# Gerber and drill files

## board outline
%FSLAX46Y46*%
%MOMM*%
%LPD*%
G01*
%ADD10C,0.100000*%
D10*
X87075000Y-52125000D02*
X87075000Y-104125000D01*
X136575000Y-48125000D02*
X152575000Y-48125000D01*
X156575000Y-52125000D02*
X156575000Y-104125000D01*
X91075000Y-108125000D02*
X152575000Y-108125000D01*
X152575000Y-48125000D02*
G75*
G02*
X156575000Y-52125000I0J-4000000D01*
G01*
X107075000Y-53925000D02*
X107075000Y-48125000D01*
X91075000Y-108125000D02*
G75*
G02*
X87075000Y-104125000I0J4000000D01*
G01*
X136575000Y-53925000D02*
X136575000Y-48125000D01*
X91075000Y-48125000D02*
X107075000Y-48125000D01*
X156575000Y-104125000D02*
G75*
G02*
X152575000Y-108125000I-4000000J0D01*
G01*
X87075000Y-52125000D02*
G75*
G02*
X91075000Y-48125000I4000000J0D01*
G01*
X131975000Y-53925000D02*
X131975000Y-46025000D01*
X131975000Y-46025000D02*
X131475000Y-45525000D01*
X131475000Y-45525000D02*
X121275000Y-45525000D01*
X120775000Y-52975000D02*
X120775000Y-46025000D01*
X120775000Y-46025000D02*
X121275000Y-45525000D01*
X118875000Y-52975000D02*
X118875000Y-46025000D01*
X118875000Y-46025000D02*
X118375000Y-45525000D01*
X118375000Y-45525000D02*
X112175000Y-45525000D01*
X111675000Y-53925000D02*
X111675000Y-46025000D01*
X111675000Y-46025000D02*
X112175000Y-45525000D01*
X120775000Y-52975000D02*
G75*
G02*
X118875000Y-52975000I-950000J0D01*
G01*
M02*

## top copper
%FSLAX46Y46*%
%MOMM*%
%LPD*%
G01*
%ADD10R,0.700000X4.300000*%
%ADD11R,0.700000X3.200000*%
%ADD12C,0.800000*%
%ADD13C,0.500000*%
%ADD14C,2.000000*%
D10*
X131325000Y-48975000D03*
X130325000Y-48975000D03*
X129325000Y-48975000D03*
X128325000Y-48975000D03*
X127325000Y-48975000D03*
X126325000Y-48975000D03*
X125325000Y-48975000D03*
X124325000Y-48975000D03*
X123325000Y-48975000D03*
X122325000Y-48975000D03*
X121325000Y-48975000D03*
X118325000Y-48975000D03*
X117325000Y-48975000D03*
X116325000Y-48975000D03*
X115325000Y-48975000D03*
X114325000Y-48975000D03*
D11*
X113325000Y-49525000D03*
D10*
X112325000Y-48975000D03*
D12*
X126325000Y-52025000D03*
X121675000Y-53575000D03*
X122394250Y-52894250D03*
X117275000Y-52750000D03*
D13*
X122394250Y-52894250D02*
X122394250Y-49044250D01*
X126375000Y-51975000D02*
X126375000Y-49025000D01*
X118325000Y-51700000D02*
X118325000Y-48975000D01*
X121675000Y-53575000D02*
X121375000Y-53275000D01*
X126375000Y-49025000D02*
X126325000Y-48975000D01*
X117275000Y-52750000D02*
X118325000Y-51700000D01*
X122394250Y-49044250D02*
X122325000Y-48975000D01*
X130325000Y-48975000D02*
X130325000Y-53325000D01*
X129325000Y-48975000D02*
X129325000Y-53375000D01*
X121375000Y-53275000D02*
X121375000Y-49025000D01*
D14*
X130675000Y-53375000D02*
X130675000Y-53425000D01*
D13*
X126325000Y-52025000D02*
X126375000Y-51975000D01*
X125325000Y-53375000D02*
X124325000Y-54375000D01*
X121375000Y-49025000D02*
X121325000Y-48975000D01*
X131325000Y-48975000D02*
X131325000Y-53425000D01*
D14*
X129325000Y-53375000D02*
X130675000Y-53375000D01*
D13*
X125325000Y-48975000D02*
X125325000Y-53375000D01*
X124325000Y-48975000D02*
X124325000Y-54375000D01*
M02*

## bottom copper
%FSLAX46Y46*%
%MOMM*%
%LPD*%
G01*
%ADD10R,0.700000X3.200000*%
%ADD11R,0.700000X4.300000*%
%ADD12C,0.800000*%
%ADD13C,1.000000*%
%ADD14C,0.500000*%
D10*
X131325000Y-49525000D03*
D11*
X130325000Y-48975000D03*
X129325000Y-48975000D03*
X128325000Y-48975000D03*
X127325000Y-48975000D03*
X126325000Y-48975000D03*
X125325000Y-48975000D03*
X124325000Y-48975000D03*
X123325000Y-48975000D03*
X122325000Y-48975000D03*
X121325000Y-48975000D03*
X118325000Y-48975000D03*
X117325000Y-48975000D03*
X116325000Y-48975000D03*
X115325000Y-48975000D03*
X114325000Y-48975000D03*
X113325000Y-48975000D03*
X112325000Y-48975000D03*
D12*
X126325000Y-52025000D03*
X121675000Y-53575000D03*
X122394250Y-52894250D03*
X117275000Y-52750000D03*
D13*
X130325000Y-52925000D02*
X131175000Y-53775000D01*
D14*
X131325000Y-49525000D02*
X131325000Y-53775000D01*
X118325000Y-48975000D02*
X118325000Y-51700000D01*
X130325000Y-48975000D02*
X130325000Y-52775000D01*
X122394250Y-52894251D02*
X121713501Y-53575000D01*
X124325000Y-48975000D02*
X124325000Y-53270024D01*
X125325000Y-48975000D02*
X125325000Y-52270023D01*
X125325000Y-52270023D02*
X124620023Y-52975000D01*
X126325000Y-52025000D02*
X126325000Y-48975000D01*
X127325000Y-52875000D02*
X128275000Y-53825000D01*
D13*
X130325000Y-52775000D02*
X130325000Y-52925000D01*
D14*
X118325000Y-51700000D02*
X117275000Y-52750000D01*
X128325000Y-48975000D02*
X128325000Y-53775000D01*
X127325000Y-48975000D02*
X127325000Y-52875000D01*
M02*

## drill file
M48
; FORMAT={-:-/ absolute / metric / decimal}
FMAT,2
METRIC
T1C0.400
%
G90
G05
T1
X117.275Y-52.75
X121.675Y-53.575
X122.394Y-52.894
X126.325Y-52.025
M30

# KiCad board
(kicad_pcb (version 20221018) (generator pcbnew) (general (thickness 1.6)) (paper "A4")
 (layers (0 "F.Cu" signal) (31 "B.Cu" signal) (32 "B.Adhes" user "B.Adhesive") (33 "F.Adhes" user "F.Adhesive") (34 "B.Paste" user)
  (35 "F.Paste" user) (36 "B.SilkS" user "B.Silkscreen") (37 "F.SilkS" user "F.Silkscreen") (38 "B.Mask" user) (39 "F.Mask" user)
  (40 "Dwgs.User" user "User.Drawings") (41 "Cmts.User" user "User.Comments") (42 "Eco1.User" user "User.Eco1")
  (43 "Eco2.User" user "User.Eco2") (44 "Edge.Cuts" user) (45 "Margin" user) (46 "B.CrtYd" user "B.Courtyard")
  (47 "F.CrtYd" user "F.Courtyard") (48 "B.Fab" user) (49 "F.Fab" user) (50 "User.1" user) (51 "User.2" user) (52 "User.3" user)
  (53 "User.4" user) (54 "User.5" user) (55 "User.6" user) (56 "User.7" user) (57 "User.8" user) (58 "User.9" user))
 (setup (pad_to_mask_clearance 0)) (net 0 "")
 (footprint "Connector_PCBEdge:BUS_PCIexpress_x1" (layer "F.Cu") (at 131.325 48.975 180)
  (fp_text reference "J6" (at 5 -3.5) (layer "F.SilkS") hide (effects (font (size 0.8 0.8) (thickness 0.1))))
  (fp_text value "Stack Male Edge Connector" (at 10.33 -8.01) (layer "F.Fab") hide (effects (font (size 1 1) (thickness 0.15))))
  (fp_line (start -0.65 -4.95) (end -0.65 2.95) (stroke (width 0.1) (type solid)) (layer "Edge.Cuts"))
  (fp_line (start -0.65 2.95) (end -0.15 3.45) (stroke (width 0.1) (type solid)) (layer "Edge.Cuts"))
  (fp_line (start -0.15 3.45) (end 10.05 3.45) (stroke (width 0.1) (type solid)) (layer "Edge.Cuts"))
  (fp_line (start 10.55 -4) (end 10.55 2.95) (stroke (width 0.1) (type solid)) (layer "Edge.Cuts"))
  (fp_line (start 10.55 2.95) (end 10.05 3.45) (stroke (width 0.1) (type solid)) (layer "Edge.Cuts"))
  (fp_line (start 12.45 -4) (end 12.45 2.95) (stroke (width 0.1) (type solid)) (layer "Edge.Cuts"))
  (fp_line (start 12.45 2.95) (end 12.95 3.45) (stroke (width 0.1) (type solid)) (layer "Edge.Cuts"))
  (fp_line (start 12.95 3.45) (end 19.15 3.45) (stroke (width 0.1) (type solid)) (layer "Edge.Cuts"))
  (fp_line (start 19.65 -4.95) (end 19.65 2.95) (stroke (width 0.1) (type solid)) (layer "Edge.Cuts"))
  (fp_line (start 19.65 2.95) (end 19.15 3.45) (stroke (width 0.1) (type solid)) (layer "Edge.Cuts"))
  (fp_arc (start 10.55 -4) (mid 11.5 -4.95) (end 12.45 -4) (stroke (width 0.1) (type solid)) (layer "Edge.Cuts"))
  (pad "A1" connect rect (at 0 -0.55 180) (size 0.7 3.2) (layers "B.Cu" "B.Mask"))
  (pad "A2" connect rect (at 1 0 180) (size 0.7 4.3) (layers "B.Cu" "B.Mask"))
  (pad "A3" connect rect (at 2 0 180) (size 0.7 4.3) (layers "B.Cu" "B.Mask"))
  (pad "A4" connect rect (at 3 0 180) (size 0.7 4.3) (layers "B.Cu" "B.Mask"))
  (pad "A5" connect rect (at 4 0 180) (size 0.7 4.3) (layers "B.Cu" "B.Mask"))
  (pad "A6" connect rect (at 5 0 180) (size 0.7 4.3) (layers "B.Cu" "B.Mask"))
  (pad "A7" connect rect (at 6 0 180) (size 0.7 4.3) (layers "B.Cu" "B.Mask"))
  (pad "A8" connect rect (at 7 0 180) (size 0.7 4.3) (layers "B.Cu" "B.Mask"))
  (pad "A9" connect rect (at 8 0 180) (size 0.7 4.3) (layers "B.Cu" "B.Mask"))
  (pad "A10" connect rect (at 9 0 180) (size 0.7 4.3) (layers "B.Cu" "B.Mask"))
  (pad "A11" connect rect (at 10 0 180) (size 0.7 4.3) (layers "B.Cu" "B.Mask"))
  (pad "A12" connect rect (at 13 0 180) (size 0.7 4.3) (layers "B.Cu" "B.Mask"))
  (pad "A13" connect rect (at 14 0 180) (size 0.7 4.3) (layers "B.Cu" "B.Mask"))
  (pad "A14" connect rect (at 15 0 180) (size 0.7 4.3) (layers "B.Cu" "B.Mask"))
  (pad "A15" connect rect (at 16 0 180) (size 0.7 4.3) (layers "B.Cu" "B.Mask"))
  (pad "A16" connect rect (at 17 0 180) (size 0.7 4.3) (layers "B.Cu" "B.Mask"))
  (pad "A17" connect rect (at 18 0 180) (size 0.7 4.3) (layers "B.Cu" "B.Mask"))
  (pad "A18" connect rect (at 19 0 180) (size 0.7 4.3) (layers "B.Cu" "B.Mask"))
  (pad "B1" connect rect (at 0 0 180) (size 0.7 4.3) (layers "F.Cu" "F.Mask"))
  (pad "B2" connect rect (at 1 0 180) (size 0.7 4.3) (layers "F.Cu" "F.Mask"))
  (pad "B3" connect rect (at 2 0 180) (size 0.7 4.3) (layers "F.Cu" "F.Mask"))
  (pad "B4" connect rect (at 3 0 180) (size 0.7 4.3) (layers "F.Cu" "F.Mask"))
  (pad "B5" connect rect (at 4 0 180) (size 0.7 4.3) (layers "F.Cu" "F.Mask"))
  (pad "B6" connect rect (at 5 0 180) (size 0.7 4.3) (layers "F.Cu" "F.Mask"))
  (pad "B7" connect rect (at 6 0 180) (size 0.7 4.3) (layers "F.Cu" "F.Mask"))
  (pad "B8" connect rect (at 7 0 180) (size 0.7 4.3) (layers "F.Cu" "F.Mask"))
  (pad "B9" connect rect (at 8 0 180) (size 0.7 4.3) (layers "F.Cu" "F.Mask"))
  (pad "B10" connect rect (at 9 0 180) (size 0.7 4.3) (layers "F.Cu" "F.Mask"))
  (pad "B11" connect rect (at 10 0 180) (size 0.7 4.3) (layers "F.Cu" "F.Mask"))
  (pad "B12" connect rect (at 13 0 180) (size 0.7 4.3) (layers "F.Cu" "F.Mask"))
  (pad "B13" connect rect (at 14 0 180) (size 0.7 4.3) (layers "F.Cu" "F.Mask"))
  (pad "B14" connect rect (at 15 0 180) (size 0.7 4.3) (layers "F.Cu" "F.Mask"))
  (pad "B15" connect rect (at 16 0 180) (size 0.7 4.3) (layers "F.Cu" "F.Mask"))
  (pad "B16" connect rect (at 17 0 180) (size 0.7 4.3) (layers "F.Cu" "F.Mask"))
  (pad "B17" connect rect (at 18 -0.55 180) (size 0.7 3.2) (layers "F.Cu" "F.Mask"))
  (pad "B18" connect rect (at 19 0 180) (size 0.7 4.3) (layers "F.Cu" "F.Mask")))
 (gr_line (start 87.075 52.125) (end 87.075 104.125) (stroke (width 0.1) (type default)) (layer "Edge.Cuts"))
 (gr_line (start 136.575 48.125) (end 152.575 48.125) (stroke (width 0.1) (type default)) (layer "Edge.Cuts"))
 (gr_line (start 156.575 52.125) (end 156.575 104.125) (stroke (width 0.1) (type default)) (layer "Edge.Cuts"))
 (gr_line (start 91.075 108.125) (end 152.575 108.125) (stroke (width 0.1) (type default)) (layer "Edge.Cuts"))
 (gr_arc (start 152.575 48.125) (mid 155.403427 49.296573) (end 156.575 52.125) (stroke (width 0.1) (type default)) (layer "Edge.Cuts"))
 (gr_line (start 107.075 53.925) (end 107.075 48.125) (stroke (width 0.1) (type default)) (layer "Edge.Cuts"))
 (gr_arc (start 91.075 108.125) (mid 88.246573 106.953427) (end 87.075 104.125) (stroke (width 0.1) (type default)) (layer "Edge.Cuts"))
 (gr_line (start 136.575 53.925) (end 136.575 48.125) (stroke (width 0.1) (type default)) (layer "Edge.Cuts"))
 (gr_line (start 91.075 48.125) (end 107.075 48.125) (stroke (width 0.1) (type default)) (layer "Edge.Cuts"))
 (gr_arc (start 156.575 104.125) (mid 155.403427 106.953427) (end 152.575 108.125) (stroke (width 0.1) (type default)) (layer "Edge.Cuts"))
 (gr_arc (start 87.075 52.125) (mid 88.246573 49.296573) (end 91.075 48.125) (stroke (width 0.1) (type default)) (layer "Edge.Cuts"))
 (segment (start 122.39425 52.89425) (end 122.39425 49.04425) (width 0.5) (layer "F.Cu") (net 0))
 (segment (start 126.375 51.975) (end 126.375 49.025) (width 0.5) (layer "F.Cu") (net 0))
 (segment (start 118.325 51.7) (end 118.325 48.975) (width 0.5) (layer "F.Cu") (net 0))
 (segment (start 121.675 53.575) (end 121.375 53.275) (width 0.5) (layer "F.Cu") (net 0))
 (segment (start 126.375 49.025) (end 126.325 48.975) (width 0.5) (layer "F.Cu") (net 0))
 (segment (start 117.275 52.75) (end 118.325 51.7) (width 0.5) (layer "F.Cu") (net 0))
 (segment (start 122.39425 49.04425) (end 122.325 48.975) (width 0.5) (layer "F.Cu") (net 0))
 (segment (start 130.325 48.975) (end 130.325 53.325) (width 0.5) (layer "F.Cu") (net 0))
 (segment (start 129.325 48.975) (end 129.325 53.375) (width 0.5) (layer "F.Cu") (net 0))
 (segment (start 121.375 53.275) (end 121.375 49.025) (width 0.5) (layer "F.Cu") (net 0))
 (segment (start 130.675 53.375) (end 130.675 53.425) (width 2) (layer "F.Cu") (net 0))
 (segment (start 126.325 52.025) (end 126.375 51.975) (width 0.5) (layer "F.Cu") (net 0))
 (segment (start 125.325 53.375) (end 124.325 54.375) (width 0.5) (layer "F.Cu") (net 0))
 (segment (start 121.375 49.025) (end 121.325 48.975) (width 0.5) (layer "F.Cu") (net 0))
 (segment (start 131.325 48.975) (end 131.325 53.425) (width 0.5) (layer "F.Cu") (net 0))
 (segment (start 129.325 53.375) (end 130.675 53.375) (width 2) (layer "F.Cu") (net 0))
 (segment (start 125.325 48.975) (end 125.325 53.375) (width 0.5) (layer "F.Cu") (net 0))
 (segment (start 124.325 48.975) (end 124.325 54.375) (width 0.5) (layer "F.Cu") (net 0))
 (via (at 126.325 52.025) (size 0.8) (drill 0.4) (layers "F.Cu" "B.Cu") (free) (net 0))
 (via (at 121.675 53.575) (size 0.8) (drill 0.4) (layers "F.Cu" "B.Cu") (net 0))
 (via (at 122.39425 52.89425) (size 0.8) (drill 0.4) (layers "F.Cu" "B.Cu") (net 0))
 (via (at 117.275 52.75) (size 0.8) (drill 0.4) (layers "F.Cu" "B.Cu") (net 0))
 (segment (start 130.325 52.925) (end 131.175 53.775) (width 1) (layer "B.Cu") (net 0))
 (segment (start 131.325 49.525) (end 131.325 53.775) (width 0.5) (layer "B.Cu") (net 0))
 (segment (start 118.325 48.975) (end 118.325 51.7) (width 0.5) (layer "B.Cu") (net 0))
 (segment (start 130.325 48.975) (end 130.325 52.775) (width 0.5) (layer "B.Cu") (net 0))
 (segment (start 122.39425 52.894251) (end 121.713501 53.575) (width 0.5) (layer "B.Cu") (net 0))
 (segment (start 124.325 48.975) (end 124.325 53.270024) (width 0.5) (layer "B.Cu") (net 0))
 (segment (start 125.325 48.975) (end 125.325 52.270023) (width 0.5) (layer "B.Cu") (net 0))
 (segment (start 125.325 52.270023) (end 124.620023 52.975) (width 0.5) (layer "B.Cu") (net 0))
 (segment (start 126.325 52.025) (end 126.325 48.975) (width 0.5) (layer "B.Cu") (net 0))
 (segment (start 127.325 52.875) (end 128.275 53.825) (width 0.5) (layer "B.Cu") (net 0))
 (segment (start 130.325 52.775) (end 130.325 52.925) (width 1) (layer "B.Cu") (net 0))
 (segment (start 118.325 51.7) (end 117.275 52.75) (width 0.5) (layer "B.Cu") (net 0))
 (segment (start 128.325 48.975) (end 128.325 53.775) (width 0.5) (layer "B.Cu") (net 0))
 (segment (start 127.325 48.975) (end 127.325 52.875) (width 0.5) (layer "B.Cu") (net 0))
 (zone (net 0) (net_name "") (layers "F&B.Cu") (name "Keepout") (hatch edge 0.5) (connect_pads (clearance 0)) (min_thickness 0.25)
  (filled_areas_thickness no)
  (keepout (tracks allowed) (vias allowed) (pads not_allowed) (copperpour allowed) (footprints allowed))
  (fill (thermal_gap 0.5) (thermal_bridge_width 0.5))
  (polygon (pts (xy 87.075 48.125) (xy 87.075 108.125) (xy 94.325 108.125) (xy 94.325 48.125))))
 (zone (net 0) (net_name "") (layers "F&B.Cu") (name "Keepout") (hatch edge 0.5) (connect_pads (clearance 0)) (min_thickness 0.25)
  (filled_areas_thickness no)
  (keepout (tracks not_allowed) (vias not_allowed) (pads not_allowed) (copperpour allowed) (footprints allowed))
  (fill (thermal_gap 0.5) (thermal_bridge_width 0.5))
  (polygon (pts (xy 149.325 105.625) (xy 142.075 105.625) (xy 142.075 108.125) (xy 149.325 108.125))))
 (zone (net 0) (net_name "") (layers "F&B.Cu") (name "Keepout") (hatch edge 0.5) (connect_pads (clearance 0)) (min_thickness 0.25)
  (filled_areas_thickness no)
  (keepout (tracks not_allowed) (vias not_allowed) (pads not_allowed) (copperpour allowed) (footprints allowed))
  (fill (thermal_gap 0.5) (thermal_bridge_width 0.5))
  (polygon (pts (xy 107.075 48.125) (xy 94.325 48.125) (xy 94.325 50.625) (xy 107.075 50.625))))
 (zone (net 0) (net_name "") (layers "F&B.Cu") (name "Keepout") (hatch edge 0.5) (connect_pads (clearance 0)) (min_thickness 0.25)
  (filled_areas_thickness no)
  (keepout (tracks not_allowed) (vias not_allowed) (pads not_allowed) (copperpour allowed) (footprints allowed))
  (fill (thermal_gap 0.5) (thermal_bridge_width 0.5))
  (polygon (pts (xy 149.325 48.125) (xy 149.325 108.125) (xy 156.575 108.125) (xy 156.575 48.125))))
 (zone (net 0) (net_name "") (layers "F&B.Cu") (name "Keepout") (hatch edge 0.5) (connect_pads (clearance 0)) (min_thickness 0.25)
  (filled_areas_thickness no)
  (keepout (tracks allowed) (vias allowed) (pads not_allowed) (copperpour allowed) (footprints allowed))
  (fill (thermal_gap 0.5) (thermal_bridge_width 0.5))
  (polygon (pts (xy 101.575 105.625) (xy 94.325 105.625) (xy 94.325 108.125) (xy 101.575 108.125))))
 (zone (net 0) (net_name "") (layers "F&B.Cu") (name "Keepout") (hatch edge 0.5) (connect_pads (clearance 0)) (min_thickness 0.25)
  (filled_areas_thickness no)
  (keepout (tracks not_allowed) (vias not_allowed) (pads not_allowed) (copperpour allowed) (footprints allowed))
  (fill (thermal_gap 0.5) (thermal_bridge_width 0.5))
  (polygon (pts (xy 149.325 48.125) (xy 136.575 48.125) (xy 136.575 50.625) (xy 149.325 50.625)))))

